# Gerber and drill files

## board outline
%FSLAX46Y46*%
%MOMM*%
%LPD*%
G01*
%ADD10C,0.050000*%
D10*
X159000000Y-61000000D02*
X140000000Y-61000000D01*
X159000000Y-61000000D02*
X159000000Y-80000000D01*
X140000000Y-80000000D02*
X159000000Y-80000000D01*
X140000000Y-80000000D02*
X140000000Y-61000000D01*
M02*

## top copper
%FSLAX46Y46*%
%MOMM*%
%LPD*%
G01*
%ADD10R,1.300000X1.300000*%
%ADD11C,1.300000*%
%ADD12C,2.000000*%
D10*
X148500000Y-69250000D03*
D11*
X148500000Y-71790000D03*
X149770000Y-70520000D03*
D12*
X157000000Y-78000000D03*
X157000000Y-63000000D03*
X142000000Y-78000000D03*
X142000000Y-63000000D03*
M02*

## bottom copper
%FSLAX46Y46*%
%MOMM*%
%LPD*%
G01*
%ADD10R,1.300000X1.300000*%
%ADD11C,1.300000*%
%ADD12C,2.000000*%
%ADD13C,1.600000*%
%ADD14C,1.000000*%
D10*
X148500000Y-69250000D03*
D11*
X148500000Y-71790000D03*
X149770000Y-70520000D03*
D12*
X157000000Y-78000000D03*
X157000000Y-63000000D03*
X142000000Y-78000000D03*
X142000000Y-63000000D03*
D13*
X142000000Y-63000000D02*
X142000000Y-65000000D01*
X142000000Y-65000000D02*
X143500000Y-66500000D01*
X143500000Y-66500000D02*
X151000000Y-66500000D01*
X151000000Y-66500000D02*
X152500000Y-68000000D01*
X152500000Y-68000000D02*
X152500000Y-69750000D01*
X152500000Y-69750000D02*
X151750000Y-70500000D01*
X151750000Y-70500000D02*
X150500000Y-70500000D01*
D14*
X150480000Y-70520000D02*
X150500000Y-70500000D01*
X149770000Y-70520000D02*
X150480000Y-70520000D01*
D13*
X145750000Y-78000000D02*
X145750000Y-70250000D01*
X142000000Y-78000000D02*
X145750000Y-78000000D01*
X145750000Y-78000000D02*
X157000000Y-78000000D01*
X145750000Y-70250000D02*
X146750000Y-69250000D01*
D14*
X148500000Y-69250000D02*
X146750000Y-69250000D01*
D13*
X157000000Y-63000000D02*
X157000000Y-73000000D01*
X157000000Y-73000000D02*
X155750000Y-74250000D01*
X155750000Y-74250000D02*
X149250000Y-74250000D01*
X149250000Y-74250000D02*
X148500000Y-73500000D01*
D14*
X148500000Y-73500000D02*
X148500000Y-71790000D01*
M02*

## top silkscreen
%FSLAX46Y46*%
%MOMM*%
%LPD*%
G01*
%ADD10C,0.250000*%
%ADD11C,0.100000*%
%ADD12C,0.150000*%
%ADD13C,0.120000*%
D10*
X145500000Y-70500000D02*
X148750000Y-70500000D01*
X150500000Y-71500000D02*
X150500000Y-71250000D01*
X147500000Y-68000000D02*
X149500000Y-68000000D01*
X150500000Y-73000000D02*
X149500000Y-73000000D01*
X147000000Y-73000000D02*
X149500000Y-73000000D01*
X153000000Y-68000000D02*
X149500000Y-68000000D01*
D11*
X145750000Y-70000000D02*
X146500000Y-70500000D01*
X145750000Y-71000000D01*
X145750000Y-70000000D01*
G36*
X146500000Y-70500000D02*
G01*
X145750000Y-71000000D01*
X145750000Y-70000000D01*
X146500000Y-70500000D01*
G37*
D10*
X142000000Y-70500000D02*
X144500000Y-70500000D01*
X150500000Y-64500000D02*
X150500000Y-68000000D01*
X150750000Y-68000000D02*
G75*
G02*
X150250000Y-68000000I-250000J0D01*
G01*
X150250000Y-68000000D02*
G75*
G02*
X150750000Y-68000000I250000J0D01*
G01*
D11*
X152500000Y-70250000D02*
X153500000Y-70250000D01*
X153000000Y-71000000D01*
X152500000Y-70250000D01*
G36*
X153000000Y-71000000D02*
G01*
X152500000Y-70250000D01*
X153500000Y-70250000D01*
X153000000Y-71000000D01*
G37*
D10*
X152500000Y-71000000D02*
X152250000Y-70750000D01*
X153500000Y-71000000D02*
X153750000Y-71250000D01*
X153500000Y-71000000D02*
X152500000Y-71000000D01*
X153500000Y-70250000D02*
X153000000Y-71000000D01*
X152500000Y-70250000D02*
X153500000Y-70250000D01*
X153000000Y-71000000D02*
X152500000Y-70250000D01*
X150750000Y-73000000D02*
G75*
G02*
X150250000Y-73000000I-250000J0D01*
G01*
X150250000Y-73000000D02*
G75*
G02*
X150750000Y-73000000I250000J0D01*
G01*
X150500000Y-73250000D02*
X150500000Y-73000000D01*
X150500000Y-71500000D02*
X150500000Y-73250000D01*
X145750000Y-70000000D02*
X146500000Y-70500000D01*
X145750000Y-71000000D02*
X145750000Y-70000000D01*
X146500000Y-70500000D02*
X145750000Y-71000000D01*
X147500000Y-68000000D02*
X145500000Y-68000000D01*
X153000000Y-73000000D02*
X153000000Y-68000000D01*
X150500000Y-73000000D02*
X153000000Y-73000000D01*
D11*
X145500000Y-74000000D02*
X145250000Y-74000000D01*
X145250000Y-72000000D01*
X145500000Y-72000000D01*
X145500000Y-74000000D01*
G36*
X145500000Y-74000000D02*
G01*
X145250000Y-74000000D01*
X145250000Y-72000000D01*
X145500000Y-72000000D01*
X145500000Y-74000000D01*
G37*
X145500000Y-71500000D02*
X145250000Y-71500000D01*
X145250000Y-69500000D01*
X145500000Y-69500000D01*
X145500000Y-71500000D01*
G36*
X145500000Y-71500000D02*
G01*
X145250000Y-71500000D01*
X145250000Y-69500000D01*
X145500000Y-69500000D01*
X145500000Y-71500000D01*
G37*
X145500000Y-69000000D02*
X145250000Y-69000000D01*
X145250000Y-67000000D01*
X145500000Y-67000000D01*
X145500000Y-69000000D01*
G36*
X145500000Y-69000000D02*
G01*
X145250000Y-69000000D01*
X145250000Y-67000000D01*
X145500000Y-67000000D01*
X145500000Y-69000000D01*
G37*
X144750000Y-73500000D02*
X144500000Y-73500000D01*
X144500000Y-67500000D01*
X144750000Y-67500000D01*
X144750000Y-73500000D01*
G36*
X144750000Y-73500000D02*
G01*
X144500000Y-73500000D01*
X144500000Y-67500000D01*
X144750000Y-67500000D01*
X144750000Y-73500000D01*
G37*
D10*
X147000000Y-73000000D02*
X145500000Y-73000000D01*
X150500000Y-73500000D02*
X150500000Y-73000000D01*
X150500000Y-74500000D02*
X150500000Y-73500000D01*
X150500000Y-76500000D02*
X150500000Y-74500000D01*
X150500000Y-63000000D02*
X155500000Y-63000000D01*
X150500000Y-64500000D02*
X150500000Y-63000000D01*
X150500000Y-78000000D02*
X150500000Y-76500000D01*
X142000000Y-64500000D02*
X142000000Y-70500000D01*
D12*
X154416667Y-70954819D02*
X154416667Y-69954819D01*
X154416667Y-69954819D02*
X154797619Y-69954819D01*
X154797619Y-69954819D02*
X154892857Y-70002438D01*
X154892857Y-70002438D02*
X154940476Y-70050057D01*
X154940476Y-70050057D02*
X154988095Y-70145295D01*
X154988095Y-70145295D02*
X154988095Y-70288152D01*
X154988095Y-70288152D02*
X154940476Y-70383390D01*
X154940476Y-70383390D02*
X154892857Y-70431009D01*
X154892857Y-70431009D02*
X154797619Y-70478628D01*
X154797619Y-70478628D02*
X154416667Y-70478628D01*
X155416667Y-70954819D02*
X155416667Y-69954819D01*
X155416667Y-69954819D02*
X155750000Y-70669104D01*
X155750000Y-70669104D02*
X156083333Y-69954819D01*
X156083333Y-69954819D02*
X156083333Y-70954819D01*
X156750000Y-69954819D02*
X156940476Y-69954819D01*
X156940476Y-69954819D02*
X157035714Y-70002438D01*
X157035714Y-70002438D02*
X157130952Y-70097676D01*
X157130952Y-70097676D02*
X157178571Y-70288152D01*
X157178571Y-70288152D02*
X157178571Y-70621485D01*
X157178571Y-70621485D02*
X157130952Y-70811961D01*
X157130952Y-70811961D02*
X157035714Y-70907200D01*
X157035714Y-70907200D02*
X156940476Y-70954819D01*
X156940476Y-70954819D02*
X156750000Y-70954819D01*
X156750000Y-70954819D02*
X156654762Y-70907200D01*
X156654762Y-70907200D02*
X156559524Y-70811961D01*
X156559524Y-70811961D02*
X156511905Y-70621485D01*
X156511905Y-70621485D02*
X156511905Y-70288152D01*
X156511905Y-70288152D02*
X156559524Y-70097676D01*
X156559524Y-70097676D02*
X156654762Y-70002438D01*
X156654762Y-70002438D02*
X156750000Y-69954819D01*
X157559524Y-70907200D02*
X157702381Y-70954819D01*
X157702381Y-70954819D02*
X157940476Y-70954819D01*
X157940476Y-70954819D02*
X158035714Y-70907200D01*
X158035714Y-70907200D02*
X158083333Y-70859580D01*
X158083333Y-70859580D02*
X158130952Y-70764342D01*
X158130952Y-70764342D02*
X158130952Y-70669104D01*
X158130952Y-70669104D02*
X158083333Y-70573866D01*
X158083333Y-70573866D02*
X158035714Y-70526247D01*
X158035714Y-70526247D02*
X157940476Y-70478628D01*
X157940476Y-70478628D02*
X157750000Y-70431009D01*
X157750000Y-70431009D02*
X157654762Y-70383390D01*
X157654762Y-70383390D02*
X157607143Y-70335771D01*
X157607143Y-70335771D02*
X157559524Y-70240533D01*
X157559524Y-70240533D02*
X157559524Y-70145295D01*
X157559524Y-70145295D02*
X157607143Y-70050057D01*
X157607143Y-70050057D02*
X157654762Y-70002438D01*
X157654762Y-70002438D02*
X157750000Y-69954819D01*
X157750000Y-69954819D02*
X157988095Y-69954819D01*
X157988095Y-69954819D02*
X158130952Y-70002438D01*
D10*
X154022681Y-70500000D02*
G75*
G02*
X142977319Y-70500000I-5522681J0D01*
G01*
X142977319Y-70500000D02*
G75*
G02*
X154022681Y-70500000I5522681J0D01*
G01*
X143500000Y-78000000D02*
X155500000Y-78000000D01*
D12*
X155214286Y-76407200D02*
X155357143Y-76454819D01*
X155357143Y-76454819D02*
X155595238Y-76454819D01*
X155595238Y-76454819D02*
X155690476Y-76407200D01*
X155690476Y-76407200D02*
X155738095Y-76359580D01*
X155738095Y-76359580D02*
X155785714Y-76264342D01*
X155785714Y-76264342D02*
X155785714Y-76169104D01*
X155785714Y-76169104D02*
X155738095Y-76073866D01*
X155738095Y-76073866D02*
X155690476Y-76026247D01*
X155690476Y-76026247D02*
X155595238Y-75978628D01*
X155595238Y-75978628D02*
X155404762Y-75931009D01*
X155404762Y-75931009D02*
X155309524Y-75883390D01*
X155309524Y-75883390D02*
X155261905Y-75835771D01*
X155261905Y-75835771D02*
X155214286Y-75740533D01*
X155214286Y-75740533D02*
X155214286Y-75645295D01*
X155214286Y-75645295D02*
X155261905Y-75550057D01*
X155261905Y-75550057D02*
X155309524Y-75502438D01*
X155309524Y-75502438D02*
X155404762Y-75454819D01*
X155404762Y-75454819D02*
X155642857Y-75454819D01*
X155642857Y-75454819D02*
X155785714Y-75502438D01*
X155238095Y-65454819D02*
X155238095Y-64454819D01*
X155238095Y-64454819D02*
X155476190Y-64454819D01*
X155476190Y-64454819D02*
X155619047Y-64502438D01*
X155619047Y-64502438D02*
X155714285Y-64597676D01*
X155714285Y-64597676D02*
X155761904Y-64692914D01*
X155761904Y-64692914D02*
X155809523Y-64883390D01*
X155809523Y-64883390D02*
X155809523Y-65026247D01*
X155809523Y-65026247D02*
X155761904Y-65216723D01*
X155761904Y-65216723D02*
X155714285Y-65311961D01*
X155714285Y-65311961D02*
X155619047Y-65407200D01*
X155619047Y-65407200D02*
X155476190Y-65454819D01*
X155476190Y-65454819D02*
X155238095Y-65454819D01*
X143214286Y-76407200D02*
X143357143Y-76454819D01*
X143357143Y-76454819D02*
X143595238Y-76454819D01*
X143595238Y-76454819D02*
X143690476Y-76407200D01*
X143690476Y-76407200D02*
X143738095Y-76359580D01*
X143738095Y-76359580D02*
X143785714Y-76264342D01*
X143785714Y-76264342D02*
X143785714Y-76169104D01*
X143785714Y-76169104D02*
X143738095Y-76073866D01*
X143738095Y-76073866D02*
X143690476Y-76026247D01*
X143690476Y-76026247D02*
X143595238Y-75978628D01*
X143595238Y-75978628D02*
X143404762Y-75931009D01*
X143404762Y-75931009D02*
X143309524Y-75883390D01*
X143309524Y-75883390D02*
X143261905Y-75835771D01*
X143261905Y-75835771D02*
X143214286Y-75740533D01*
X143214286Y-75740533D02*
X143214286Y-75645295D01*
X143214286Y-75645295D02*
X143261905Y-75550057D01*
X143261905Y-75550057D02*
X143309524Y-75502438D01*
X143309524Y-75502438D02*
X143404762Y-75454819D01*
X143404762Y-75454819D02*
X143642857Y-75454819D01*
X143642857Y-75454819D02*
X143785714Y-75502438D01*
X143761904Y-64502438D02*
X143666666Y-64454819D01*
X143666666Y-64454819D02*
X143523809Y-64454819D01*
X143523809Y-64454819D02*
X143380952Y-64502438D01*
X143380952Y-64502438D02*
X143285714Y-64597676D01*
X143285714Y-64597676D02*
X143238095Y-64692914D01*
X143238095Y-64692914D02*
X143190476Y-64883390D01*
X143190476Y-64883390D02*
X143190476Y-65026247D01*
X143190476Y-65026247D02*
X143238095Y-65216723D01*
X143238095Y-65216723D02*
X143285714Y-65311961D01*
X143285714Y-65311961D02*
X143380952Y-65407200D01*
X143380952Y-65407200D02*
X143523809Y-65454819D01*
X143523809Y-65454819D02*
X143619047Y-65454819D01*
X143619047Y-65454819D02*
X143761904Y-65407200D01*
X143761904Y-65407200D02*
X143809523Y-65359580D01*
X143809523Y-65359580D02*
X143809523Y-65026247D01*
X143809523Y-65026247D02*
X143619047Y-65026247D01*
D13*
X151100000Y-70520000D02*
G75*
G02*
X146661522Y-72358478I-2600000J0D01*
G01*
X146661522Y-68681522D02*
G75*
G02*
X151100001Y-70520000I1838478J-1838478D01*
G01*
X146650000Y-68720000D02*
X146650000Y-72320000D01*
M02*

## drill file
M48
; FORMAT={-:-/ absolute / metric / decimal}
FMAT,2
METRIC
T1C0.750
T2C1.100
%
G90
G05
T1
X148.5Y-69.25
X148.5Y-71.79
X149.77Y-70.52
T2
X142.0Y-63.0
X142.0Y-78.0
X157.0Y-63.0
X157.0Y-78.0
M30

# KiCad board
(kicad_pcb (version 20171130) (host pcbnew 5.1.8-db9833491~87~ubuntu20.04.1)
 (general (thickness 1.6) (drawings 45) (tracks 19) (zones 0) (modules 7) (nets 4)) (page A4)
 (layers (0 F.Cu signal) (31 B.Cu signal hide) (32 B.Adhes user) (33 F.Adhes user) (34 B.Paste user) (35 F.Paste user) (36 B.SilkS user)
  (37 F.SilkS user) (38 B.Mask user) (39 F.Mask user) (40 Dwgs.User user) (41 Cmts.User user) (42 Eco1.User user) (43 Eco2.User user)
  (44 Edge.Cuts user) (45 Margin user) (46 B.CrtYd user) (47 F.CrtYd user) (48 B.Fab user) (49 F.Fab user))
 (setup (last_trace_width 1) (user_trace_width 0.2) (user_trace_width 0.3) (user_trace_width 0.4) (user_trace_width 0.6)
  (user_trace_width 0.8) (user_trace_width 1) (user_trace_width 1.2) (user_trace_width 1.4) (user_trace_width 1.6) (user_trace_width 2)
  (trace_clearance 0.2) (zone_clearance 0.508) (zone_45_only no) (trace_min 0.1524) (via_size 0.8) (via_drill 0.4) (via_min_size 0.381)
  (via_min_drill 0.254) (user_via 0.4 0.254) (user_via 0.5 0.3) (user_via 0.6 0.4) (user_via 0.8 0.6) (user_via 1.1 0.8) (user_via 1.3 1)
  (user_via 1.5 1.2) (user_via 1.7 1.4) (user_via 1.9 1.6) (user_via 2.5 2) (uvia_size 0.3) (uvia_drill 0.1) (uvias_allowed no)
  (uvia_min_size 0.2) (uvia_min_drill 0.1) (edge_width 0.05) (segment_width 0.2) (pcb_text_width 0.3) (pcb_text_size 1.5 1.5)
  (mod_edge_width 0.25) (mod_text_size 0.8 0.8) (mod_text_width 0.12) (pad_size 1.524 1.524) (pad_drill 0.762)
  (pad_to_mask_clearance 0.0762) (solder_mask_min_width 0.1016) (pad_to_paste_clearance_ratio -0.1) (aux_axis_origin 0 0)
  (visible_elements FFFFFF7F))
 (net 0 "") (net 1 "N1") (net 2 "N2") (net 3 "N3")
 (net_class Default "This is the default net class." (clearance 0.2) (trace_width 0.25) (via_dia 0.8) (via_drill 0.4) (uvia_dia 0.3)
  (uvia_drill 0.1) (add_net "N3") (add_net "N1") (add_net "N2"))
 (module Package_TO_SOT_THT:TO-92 (layer F.Cu) (at 148.5 69.25 270)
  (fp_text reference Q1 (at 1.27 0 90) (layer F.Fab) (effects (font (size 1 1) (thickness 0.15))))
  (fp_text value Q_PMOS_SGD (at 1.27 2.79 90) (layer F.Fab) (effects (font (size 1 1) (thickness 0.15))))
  (fp_arc (start 1.27 0) (end 1.27 -2.6) (angle 135) (layer F.SilkS) (width 0.12))
  (fp_arc (start 1.27 0) (end 1.27 -2.6) (angle -135) (layer F.SilkS) (width 0.12))
  (fp_line (start -0.53 1.85) (end 3.07 1.85) (layer F.SilkS) (width 0.12))
  (pad 1 thru_hole rect (at 0 0 270) (size 1.3 1.3) (drill 0.75) (layers *.Cu *.Mask) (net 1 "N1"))
  (pad 3 thru_hole circle (at 2.54 0 270) (size 1.3 1.3) (drill 0.75) (layers *.Cu *.Mask) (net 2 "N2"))
  (pad 2 thru_hole circle (at 1.27 -1.27 270) (size 1.3 1.3) (drill 0.75) (layers *.Cu *.Mask) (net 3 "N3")))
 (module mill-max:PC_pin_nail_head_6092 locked (layer F.Cu) (at 157 78)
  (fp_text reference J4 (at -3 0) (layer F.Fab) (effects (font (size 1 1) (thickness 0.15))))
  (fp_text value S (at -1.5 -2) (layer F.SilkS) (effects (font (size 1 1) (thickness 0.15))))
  (pad 1 thru_hole circle (at 0 0) (size 2 2) (drill 1.1) (layers *.Cu *.Mask) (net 1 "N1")))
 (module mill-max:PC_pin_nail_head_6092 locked (layer F.Cu) (at 157 63)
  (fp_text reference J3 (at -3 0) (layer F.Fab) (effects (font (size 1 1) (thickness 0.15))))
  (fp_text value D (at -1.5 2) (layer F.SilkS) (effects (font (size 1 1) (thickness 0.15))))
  (pad 1 thru_hole circle (at 0 0) (size 2 2) (drill 1.1) (layers *.Cu *.Mask) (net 2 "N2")))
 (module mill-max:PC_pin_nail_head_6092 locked (layer F.Cu) (at 142 78)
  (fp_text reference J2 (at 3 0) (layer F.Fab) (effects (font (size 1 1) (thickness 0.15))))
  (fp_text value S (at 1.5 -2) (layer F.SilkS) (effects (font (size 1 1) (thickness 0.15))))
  (pad 1 thru_hole circle (at 0 0) (size 2 2) (drill 1.1) (layers *.Cu *.Mask) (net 1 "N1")))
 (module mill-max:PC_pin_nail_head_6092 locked (layer F.Cu) (at 142 63)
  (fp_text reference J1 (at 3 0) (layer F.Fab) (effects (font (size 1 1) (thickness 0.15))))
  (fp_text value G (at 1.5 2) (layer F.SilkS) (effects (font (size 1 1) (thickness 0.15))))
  (pad 1 thru_hole circle (at 0 0) (size 2 2) (drill 1.1) (layers *.Cu *.Mask) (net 3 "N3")))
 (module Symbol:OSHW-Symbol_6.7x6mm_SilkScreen (layer B.Cu) (at 153.75 70.5 270)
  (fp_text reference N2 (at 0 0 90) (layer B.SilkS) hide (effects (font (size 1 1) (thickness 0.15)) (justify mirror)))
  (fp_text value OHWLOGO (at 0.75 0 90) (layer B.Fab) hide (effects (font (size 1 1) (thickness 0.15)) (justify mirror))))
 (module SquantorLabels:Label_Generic (layer B.Cu) (at 157.5 71.5 90)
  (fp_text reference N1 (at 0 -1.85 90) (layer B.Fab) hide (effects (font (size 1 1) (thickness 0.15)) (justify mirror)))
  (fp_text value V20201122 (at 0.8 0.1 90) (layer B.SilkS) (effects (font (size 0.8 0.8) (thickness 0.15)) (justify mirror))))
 (gr_line (start 145.5 70.5) (end 148.75 70.5) (layer F.SilkS) (width 0.25))
 (gr_line (start 150.5 71.5) (end 150.5 71.25) (layer F.SilkS) (width 0.25))
 (gr_line (start 147.5 68) (end 149.5 68) (layer F.SilkS) (width 0.25))
 (gr_line (start 150.5 73) (end 149.5 73) (layer F.SilkS) (width 0.25))
 (gr_line (start 147 73) (end 149.5 73) (layer F.SilkS) (width 0.25))
 (gr_line (start 153 68) (end 149.5 68) (layer F.SilkS) (width 0.25))
 (gr_poly (pts (xy 145.75 70) (xy 146.5 70.5) (xy 145.75 71)) (layer F.SilkS) (width 0.1))
 (gr_line (start 142 70.5) (end 144.5 70.5) (layer F.SilkS) (width 0.25))
 (gr_line (start 150.5 64.5) (end 150.5 68) (layer F.SilkS) (width 0.25))
 (gr_circle (center 150.5 68) (end 150.75 68) (layer F.SilkS) (width 0.25))
 (gr_poly (pts (xy 152.5 70.25) (xy 153.5 70.25) (xy 153 71)) (layer F.SilkS) (width 0.1))
 (gr_line (start 152.5 71) (end 152.25 70.75) (layer F.SilkS) (width 0.25))
 (gr_line (start 153.5 71) (end 153.75 71.25) (layer F.SilkS) (width 0.25))
 (gr_line (start 153.5 71) (end 152.5 71) (layer F.SilkS) (width 0.25))
 (gr_line (start 153.5 70.25) (end 153 71) (layer F.SilkS) (width 0.25))
 (gr_line (start 152.5 70.25) (end 153.5 70.25) (layer F.SilkS) (width 0.25))
 (gr_line (start 153 71) (end 152.5 70.25) (layer F.SilkS) (width 0.25))
 (gr_circle (center 150.5 73) (end 150.75 73) (layer F.SilkS) (width 0.25))
 (gr_line (start 150.5 73.25) (end 150.5 73) (layer F.SilkS) (width 0.25))
 (gr_line (start 150.5 71.5) (end 150.5 73.25) (layer F.SilkS) (width 0.25))
 (gr_line (start 145.75 70) (end 146.5 70.5) (layer F.SilkS) (width 0.25))
 (gr_line (start 145.75 71) (end 145.75 70) (layer F.SilkS) (width 0.25))
 (gr_line (start 146.5 70.5) (end 145.75 71) (layer F.SilkS) (width 0.25))
 (gr_line (start 147.5 68) (end 145.5 68) (layer F.SilkS) (width 0.25))
 (gr_line (start 153 73) (end 153 68) (layer F.SilkS) (width 0.25))
 (gr_line (start 150.5 73) (end 153 73) (layer F.SilkS) (width 0.25))
 (gr_poly (pts (xy 145.5 74) (xy 145.25 74) (xy 145.25 72) (xy 145.5 72)) (layer F.SilkS) (width 0.1))
 (gr_poly (pts (xy 145.5 71.5) (xy 145.25 71.5) (xy 145.25 69.5) (xy 145.5 69.5)) (layer F.SilkS) (width 0.1))
 (gr_poly (pts (xy 145.5 69) (xy 145.25 69) (xy 145.25 67) (xy 145.5 67)) (layer F.SilkS) (width 0.1))
 (gr_poly (pts (xy 144.75 73.5) (xy 144.5 73.5) (xy 144.5 67.5) (xy 144.75 67.5)) (layer F.SilkS) (width 0.1))
 (gr_line (start 147 73) (end 145.5 73) (layer F.SilkS) (width 0.25))
 (gr_line (start 150.5 73.5) (end 150.5 73) (layer F.SilkS) (width 0.25))
 (gr_line (start 150.5 74.5) (end 150.5 73.5) (layer F.SilkS) (width 0.25))
 (gr_line (start 150.5 76.5) (end 150.5 74.5) (layer F.SilkS) (width 0.25))
 (gr_line (start 150.5 63) (end 155.5 63) (layer F.SilkS) (width 0.25))
 (gr_line (start 150.5 64.5) (end 150.5 63) (layer F.SilkS) (width 0.25))
 (gr_line (start 150.5 78) (end 150.5 76.5) (layer F.SilkS) (width 0.25))
 (gr_line (start 142 64.5) (end 142 70.5) (layer F.SilkS) (width 0.25))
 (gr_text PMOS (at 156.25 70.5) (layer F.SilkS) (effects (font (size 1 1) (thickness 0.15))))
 (gr_circle (center 148.5 70.5) (end 154 71) (layer F.SilkS) (width 0.25))
 (gr_line (start 143.5 78) (end 155.5 78) (layer F.SilkS) (width 0.25))
 (gr_line (start 159 61) (end 140 61) (layer Edge.Cuts) (width 0.05))
 (gr_line (start 159 61) (end 159 80) (layer Edge.Cuts) (width 0.05))
 (gr_line (start 140 80) (end 159 80) (layer Edge.Cuts) (width 0.05))
 (gr_line (start 140 80) (end 140 61) (layer Edge.Cuts) (width 0.05))
 (segment (start 142 63) (end 142 65) (width 1.6) (layer B.Cu) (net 3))
 (segment (start 142 65) (end 143.5 66.5) (width 1.6) (layer B.Cu) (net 3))
 (segment (start 143.5 66.5) (end 151 66.5) (width 1.6) (layer B.Cu) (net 3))
 (segment (start 151 66.5) (end 152.5 68) (width 1.6) (layer B.Cu) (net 3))
 (segment (start 152.5 68) (end 152.5 69.75) (width 1.6) (layer B.Cu) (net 3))
 (segment (start 152.5 69.75) (end 151.75 70.5) (width 1.6) (layer B.Cu) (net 3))
 (segment (start 151.75 70.5) (end 150.5 70.5) (width 1.6) (layer B.Cu) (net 3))
 (segment (start 150.48 70.52) (end 150.5 70.5) (width 1) (layer B.Cu) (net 3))
 (segment (start 149.77 70.52) (end 150.48 70.52) (width 1) (layer B.Cu) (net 3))
 (segment (start 145.75 78) (end 145.75 70.25) (width 1.6) (layer B.Cu) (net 1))
 (segment (start 142 78) (end 145.75 78) (width 1.6) (layer B.Cu) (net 1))
 (segment (start 145.75 78) (end 157 78) (width 1.6) (layer B.Cu) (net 1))
 (segment (start 145.75 70.25) (end 146.75 69.25) (width 1.6) (layer B.Cu) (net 1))
 (segment (start 148.5 69.25) (end 146.75 69.25) (width 1) (layer B.Cu) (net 1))
 (segment (start 157 63) (end 157 73) (width 1.6) (layer B.Cu) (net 2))
 (segment (start 157 73) (end 155.75 74.25) (width 1.6) (layer B.Cu) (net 2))
 (segment (start 155.75 74.25) (end 149.25 74.25) (width 1.6) (layer B.Cu) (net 2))
 (segment (start 149.25 74.25) (end 148.5 73.5) (width 1.6) (layer B.Cu) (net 2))
 (segment (start 148.5 73.5) (end 148.5 71.79) (width 1) (layer B.Cu) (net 2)))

